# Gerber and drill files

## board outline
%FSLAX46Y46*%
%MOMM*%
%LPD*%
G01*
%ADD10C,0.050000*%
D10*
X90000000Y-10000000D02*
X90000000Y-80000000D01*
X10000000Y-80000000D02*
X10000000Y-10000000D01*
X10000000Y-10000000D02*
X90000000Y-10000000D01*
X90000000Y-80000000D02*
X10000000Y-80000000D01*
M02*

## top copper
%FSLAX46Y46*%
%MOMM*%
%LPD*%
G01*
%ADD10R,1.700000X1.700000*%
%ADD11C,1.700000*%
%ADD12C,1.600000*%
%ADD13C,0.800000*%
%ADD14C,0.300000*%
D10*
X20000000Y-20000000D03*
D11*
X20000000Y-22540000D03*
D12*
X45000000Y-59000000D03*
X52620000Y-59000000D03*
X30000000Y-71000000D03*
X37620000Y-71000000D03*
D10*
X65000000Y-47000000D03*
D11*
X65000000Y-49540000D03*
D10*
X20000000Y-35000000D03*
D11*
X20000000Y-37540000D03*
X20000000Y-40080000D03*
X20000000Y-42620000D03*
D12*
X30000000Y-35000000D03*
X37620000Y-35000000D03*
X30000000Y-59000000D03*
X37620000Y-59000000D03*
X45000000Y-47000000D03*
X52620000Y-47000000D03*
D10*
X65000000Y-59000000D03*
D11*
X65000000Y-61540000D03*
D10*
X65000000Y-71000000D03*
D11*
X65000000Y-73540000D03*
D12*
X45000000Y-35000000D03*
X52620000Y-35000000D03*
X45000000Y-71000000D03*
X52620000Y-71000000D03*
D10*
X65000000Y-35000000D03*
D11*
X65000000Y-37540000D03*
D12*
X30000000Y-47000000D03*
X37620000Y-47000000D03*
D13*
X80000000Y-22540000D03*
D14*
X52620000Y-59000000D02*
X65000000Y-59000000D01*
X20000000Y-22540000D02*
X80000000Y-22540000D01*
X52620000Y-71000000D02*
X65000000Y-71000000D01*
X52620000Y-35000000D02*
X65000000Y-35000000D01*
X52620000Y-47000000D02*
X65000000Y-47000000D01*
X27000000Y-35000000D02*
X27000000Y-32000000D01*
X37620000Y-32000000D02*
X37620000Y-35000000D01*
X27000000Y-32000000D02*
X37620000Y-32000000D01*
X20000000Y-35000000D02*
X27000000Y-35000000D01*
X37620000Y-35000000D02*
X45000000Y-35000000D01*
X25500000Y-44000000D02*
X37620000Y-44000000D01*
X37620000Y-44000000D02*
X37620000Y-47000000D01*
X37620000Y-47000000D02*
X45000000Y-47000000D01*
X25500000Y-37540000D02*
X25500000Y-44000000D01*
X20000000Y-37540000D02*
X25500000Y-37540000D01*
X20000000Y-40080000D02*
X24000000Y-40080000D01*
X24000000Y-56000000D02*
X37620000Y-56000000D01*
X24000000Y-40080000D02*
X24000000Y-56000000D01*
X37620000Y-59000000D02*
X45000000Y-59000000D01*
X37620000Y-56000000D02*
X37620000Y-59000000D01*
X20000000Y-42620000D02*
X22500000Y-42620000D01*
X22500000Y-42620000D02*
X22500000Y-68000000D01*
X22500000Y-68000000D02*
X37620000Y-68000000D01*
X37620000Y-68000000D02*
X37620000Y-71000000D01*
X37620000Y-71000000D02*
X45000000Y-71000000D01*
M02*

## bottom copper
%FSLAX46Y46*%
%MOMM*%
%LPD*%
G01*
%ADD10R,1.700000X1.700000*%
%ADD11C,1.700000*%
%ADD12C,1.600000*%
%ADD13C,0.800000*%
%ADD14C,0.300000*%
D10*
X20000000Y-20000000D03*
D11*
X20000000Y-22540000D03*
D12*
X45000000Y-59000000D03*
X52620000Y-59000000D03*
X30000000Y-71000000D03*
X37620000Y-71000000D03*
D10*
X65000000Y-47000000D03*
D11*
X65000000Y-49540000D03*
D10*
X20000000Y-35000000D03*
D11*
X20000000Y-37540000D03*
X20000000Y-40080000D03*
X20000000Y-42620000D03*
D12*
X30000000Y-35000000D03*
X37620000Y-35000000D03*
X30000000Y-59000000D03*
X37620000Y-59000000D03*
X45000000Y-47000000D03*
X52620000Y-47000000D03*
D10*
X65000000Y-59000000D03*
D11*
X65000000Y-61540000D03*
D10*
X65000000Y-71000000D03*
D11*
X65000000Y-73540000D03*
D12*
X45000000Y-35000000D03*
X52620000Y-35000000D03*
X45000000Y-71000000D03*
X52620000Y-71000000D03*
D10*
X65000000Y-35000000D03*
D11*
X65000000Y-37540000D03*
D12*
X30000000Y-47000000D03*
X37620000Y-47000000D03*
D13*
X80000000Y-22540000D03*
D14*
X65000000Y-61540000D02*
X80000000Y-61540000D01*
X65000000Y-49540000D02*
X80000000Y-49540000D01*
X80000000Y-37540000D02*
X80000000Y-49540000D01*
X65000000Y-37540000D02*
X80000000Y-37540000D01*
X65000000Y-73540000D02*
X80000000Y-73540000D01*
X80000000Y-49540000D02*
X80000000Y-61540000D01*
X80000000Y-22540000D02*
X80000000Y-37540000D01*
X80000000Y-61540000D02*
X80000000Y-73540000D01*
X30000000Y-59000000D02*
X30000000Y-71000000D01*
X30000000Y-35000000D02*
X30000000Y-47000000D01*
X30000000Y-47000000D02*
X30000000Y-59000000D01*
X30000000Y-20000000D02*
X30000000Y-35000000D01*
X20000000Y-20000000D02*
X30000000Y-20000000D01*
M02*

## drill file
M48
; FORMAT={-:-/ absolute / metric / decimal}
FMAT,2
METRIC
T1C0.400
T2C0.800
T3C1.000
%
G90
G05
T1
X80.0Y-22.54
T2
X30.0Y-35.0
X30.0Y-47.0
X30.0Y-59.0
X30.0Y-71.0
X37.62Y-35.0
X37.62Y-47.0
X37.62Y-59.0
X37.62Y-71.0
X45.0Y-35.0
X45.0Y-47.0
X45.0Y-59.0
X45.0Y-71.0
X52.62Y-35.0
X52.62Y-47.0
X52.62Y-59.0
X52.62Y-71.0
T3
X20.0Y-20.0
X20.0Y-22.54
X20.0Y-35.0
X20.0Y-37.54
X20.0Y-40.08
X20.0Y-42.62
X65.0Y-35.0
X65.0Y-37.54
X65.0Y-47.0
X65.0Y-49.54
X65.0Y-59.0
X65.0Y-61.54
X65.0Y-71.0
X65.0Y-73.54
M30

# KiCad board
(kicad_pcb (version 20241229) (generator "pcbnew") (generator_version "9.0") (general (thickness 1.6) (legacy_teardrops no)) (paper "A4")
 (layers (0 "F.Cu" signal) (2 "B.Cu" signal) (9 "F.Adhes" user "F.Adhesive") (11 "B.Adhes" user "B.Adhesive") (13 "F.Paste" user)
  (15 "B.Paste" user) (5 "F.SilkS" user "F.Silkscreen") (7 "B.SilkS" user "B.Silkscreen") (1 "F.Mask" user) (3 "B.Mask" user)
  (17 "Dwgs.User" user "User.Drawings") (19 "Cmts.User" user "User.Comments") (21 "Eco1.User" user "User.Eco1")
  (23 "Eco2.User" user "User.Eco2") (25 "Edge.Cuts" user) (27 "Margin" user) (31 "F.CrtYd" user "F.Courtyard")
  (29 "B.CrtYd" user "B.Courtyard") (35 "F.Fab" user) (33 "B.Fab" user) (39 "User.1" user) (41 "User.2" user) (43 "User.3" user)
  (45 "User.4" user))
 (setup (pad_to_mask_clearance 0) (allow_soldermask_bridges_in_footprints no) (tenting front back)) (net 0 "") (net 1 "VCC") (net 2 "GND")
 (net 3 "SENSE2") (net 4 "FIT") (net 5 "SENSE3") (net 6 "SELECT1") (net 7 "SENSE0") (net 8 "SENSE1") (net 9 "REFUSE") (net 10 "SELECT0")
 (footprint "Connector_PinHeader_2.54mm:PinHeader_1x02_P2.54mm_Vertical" (layer "F.Cu") (at 20 20)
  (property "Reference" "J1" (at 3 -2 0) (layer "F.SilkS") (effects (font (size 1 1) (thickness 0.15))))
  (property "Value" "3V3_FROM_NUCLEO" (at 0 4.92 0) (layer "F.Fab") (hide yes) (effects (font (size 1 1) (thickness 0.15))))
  (pad "1" thru_hole rect (at 0 0) (size 1.7 1.7) (drill 1) (layers "*.Cu" "*.Mask") (remove_unused_layers no) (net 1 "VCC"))
  (pad "2" thru_hole circle (at 0 2.54) (size 1.7 1.7) (drill 1) (layers "*.Cu" "*.Mask") (remove_unused_layers no) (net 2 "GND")))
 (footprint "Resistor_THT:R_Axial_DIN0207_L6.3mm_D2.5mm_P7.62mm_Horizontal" (layer "F.Cu") (at 45 59)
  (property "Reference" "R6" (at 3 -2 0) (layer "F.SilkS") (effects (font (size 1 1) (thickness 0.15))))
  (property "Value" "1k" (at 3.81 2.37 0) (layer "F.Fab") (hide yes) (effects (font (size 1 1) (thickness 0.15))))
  (pad "1" thru_hole circle (at 0 0) (size 1.6 1.6) (drill 0.8) (layers "*.Cu" "*.Mask") (remove_unused_layers no) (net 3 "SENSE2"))
  (pad "2" thru_hole circle (at 7.62 0) (size 1.6 1.6) (drill 0.8) (layers "*.Cu" "*.Mask") (remove_unused_layers no) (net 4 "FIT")))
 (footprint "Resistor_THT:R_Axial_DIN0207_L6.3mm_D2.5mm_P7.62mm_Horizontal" (layer "F.Cu") (at 30 71)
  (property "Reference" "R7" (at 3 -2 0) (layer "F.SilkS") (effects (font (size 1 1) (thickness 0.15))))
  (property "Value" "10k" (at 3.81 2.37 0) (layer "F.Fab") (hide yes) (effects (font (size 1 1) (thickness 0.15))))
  (pad "1" thru_hole circle (at 0 0) (size 1.6 1.6) (drill 0.8) (layers "*.Cu" "*.Mask") (remove_unused_layers no) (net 1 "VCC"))
  (pad "2" thru_hole circle (at 7.62 0) (size 1.6 1.6) (drill 0.8) (layers "*.Cu" "*.Mask") (remove_unused_layers no) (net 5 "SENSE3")))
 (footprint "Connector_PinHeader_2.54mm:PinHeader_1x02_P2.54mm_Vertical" (layer "F.Cu") (at 65 47)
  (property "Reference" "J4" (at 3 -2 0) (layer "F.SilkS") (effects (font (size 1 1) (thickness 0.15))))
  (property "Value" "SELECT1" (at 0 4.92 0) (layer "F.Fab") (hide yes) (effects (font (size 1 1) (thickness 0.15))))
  (pad "1" thru_hole rect (at 0 0) (size 1.7 1.7) (drill 1) (layers "*.Cu" "*.Mask") (remove_unused_layers no) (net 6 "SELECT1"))
  (pad "2" thru_hole circle (at 0 2.54) (size 1.7 1.7) (drill 1) (layers "*.Cu" "*.Mask") (remove_unused_layers no) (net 2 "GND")))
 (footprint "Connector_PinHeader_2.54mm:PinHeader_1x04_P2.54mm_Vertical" (layer "F.Cu") (at 20 35)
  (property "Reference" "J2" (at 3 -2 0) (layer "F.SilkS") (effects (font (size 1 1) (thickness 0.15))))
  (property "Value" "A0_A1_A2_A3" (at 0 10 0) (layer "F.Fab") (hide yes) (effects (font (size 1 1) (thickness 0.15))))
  (pad "1" thru_hole rect (at 0 0) (size 1.7 1.7) (drill 1) (layers "*.Cu" "*.Mask") (remove_unused_layers no) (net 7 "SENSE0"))
  (pad "2" thru_hole circle (at 0 2.54) (size 1.7 1.7) (drill 1) (layers "*.Cu" "*.Mask") (remove_unused_layers no) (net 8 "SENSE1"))
  (pad "3" thru_hole circle (at 0 5.08) (size 1.7 1.7) (drill 1) (layers "*.Cu" "*.Mask") (remove_unused_layers no) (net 3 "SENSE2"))
  (pad "4" thru_hole circle (at 0 7.62) (size 1.7 1.7) (drill 1) (layers "*.Cu" "*.Mask") (remove_unused_layers no) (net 5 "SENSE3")))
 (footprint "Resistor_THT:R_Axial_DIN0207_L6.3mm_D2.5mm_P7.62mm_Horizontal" (layer "F.Cu") (at 30 35)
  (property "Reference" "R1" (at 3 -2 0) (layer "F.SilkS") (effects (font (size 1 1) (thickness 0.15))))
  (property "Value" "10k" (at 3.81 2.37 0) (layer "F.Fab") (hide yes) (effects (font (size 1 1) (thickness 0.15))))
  (pad "1" thru_hole circle (at 0 0) (size 1.6 1.6) (drill 0.8) (layers "*.Cu" "*.Mask") (remove_unused_layers no) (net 1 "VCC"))
  (pad "2" thru_hole circle (at 7.62 0) (size 1.6 1.6) (drill 0.8) (layers "*.Cu" "*.Mask") (remove_unused_layers no) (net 7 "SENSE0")))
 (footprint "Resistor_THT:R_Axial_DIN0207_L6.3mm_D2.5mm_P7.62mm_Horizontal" (layer "F.Cu") (at 30 59)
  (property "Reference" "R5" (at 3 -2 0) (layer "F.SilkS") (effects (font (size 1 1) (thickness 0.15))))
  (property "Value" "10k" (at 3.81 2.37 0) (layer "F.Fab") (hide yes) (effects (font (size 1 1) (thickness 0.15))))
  (pad "1" thru_hole circle (at 0 0) (size 1.6 1.6) (drill 0.8) (layers "*.Cu" "*.Mask") (remove_unused_layers no) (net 1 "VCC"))
  (pad "2" thru_hole circle (at 7.62 0) (size 1.6 1.6) (drill 0.8) (layers "*.Cu" "*.Mask") (remove_unused_layers no) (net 3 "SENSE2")))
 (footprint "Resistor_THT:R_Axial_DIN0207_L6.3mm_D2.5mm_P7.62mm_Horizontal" (layer "F.Cu") (at 45 47)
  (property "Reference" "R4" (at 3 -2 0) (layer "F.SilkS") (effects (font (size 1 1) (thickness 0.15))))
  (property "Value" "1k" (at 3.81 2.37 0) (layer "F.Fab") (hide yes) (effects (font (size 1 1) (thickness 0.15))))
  (pad "1" thru_hole circle (at 0 0) (size 1.6 1.6) (drill 0.8) (layers "*.Cu" "*.Mask") (remove_unused_layers no) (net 8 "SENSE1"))
  (pad "2" thru_hole circle (at 7.62 0) (size 1.6 1.6) (drill 0.8) (layers "*.Cu" "*.Mask") (remove_unused_layers no) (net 6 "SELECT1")))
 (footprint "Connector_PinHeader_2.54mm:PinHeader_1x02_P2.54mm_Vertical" (layer "F.Cu") (at 65 59)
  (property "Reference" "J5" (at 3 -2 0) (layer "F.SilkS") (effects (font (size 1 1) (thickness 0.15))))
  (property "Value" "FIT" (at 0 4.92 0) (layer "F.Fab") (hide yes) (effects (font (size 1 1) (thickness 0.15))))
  (pad "1" thru_hole rect (at 0 0) (size 1.7 1.7) (drill 1) (layers "*.Cu" "*.Mask") (remove_unused_layers no) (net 4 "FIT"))
  (pad "2" thru_hole circle (at 0 2.54) (size 1.7 1.7) (drill 1) (layers "*.Cu" "*.Mask") (remove_unused_layers no) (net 2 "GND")))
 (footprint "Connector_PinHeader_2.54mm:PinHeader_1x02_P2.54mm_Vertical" (layer "F.Cu") (at 65 71)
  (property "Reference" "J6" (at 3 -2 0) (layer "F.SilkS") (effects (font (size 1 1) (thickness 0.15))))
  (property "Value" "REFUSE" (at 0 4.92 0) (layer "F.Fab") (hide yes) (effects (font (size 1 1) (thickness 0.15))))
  (pad "1" thru_hole rect (at 0 0) (size 1.7 1.7) (drill 1) (layers "*.Cu" "*.Mask") (remove_unused_layers no) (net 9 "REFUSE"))
  (pad "2" thru_hole circle (at 0 2.54) (size 1.7 1.7) (drill 1) (layers "*.Cu" "*.Mask") (remove_unused_layers no) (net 2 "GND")))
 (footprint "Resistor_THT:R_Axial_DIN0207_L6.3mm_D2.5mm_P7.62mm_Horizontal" (layer "F.Cu") (at 45 35)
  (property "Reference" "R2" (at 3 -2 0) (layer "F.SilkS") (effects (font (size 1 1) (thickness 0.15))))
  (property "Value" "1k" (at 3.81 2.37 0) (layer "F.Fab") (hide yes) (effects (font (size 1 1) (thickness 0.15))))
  (pad "1" thru_hole circle (at 0 0) (size 1.6 1.6) (drill 0.8) (layers "*.Cu" "*.Mask") (remove_unused_layers no) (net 7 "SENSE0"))
  (pad "2" thru_hole circle (at 7.62 0) (size 1.6 1.6) (drill 0.8) (layers "*.Cu" "*.Mask") (remove_unused_layers no) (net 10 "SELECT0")))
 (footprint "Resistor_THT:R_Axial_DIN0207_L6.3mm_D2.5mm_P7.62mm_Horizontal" (layer "F.Cu") (at 45 71)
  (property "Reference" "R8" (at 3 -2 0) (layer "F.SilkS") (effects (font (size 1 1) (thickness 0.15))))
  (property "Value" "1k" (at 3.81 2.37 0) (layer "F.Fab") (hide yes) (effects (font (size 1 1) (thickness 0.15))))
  (pad "1" thru_hole circle (at 0 0) (size 1.6 1.6) (drill 0.8) (layers "*.Cu" "*.Mask") (remove_unused_layers no) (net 5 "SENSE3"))
  (pad "2" thru_hole circle (at 7.62 0) (size 1.6 1.6) (drill 0.8) (layers "*.Cu" "*.Mask") (remove_unused_layers no) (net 9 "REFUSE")))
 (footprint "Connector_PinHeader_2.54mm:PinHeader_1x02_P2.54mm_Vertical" (layer "F.Cu") (at 65 35)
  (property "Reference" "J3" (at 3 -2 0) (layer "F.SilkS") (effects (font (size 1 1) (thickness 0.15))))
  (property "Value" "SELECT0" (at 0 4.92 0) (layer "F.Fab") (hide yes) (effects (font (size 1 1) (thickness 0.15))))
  (pad "1" thru_hole rect (at 0 0) (size 1.7 1.7) (drill 1) (layers "*.Cu" "*.Mask") (remove_unused_layers no) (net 10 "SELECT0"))
  (pad "2" thru_hole circle (at 0 2.54) (size 1.7 1.7) (drill 1) (layers "*.Cu" "*.Mask") (remove_unused_layers no) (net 2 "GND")))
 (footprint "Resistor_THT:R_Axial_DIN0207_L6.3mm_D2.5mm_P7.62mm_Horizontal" (layer "F.Cu") (at 30 47)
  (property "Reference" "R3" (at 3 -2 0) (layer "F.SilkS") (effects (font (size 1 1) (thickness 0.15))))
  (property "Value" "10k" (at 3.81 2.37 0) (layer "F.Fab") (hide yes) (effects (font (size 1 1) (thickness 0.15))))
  (pad "1" thru_hole circle (at 0 0) (size 1.6 1.6) (drill 0.8) (layers "*.Cu" "*.Mask") (remove_unused_layers no) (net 1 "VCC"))
  (pad "2" thru_hole circle (at 7.62 0) (size 1.6 1.6) (drill 0.8) (layers "*.Cu" "*.Mask") (remove_unused_layers no) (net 8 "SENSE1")))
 (gr_line (start 90 10) (end 90 80) (stroke (width 0.05) (type default)) (layer "Edge.Cuts"))
 (gr_line (start 10 80) (end 10 10) (stroke (width 0.05) (type default)) (layer "Edge.Cuts"))
 (gr_line (start 10 10) (end 90 10) (stroke (width 0.05) (type default)) (layer "Edge.Cuts"))
 (gr_line (start 90 80) (end 10 80) (stroke (width 0.05) (type default)) (layer "Edge.Cuts"))
 (segment (start 52.62 59) (end 65 59) (width 0.3) (layer "F.Cu") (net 4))
 (segment (start 20 22.54) (end 80 22.54) (width 0.3) (layer "F.Cu") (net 2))
 (via (at 80 22.54) (size 0.8) (drill 0.4) (layers "F.Cu" "B.Cu") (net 2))
 (segment (start 65 61.54) (end 80 61.54) (width 0.3) (layer "B.Cu") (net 2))
 (segment (start 65 49.54) (end 80 49.54) (width 0.3) (layer "B.Cu") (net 2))
 (segment (start 80 37.54) (end 80 49.54) (width 0.3) (layer "B.Cu") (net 2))
 (segment (start 65 37.54) (end 80 37.54) (width 0.3) (layer "B.Cu") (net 2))
 (segment (start 65 73.54) (end 80 73.54) (width 0.3) (layer "B.Cu") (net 2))
 (segment (start 80 49.54) (end 80 61.54) (width 0.3) (layer "B.Cu") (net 2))
 (segment (start 80 22.54) (end 80 37.54) (width 0.3) (layer "B.Cu") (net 2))
 (segment (start 80 61.54) (end 80 73.54) (width 0.3) (layer "B.Cu") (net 2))
 (segment (start 52.62 71) (end 65 71) (width 0.3) (layer "F.Cu") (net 9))
 (segment (start 52.62 35) (end 65 35) (width 0.3) (layer "F.Cu") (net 10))
 (segment (start 52.62 47) (end 65 47) (width 0.3) (layer "F.Cu") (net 6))
 (segment (start 27 35) (end 27 32) (width 0.3) (layer "F.Cu") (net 7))
 (segment (start 37.62 32) (end 37.62 35) (width 0.3) (layer "F.Cu") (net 7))
 (segment (start 27 32) (end 37.62 32) (width 0.3) (layer "F.Cu") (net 7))
 (segment (start 20 35) (end 27 35) (width 0.3) (layer "F.Cu") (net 7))
 (segment (start 37.62 35) (end 45 35) (width 0.3) (layer "F.Cu") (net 7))
 (segment (start 25.5 44) (end 37.62 44) (width 0.3) (layer "F.Cu") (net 8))
 (segment (start 37.62 44) (end 37.62 47) (width 0.3) (layer "F.Cu") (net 8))
 (segment (start 37.62 47) (end 45 47) (width 0.3) (layer "F.Cu") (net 8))
 (segment (start 25.5 37.54) (end 25.5 44) (width 0.3) (layer "F.Cu") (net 8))
 (segment (start 20 37.54) (end 25.5 37.54) (width 0.3) (layer "F.Cu") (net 8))
 (segment (start 20 40.08) (end 24 40.08) (width 0.3) (layer "F.Cu") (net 3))
 (segment (start 24 56) (end 37.62 56) (width 0.3) (layer "F.Cu") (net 3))
 (segment (start 24 40.08) (end 24 56) (width 0.3) (layer "F.Cu") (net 3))
 (segment (start 37.62 59) (end 45 59) (width 0.3) (layer "F.Cu") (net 3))
 (segment (start 37.62 56) (end 37.62 59) (width 0.3) (layer "F.Cu") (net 3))
 (segment (start 20 42.62) (end 22.5 42.62) (width 0.3) (layer "F.Cu") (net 5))
 (segment (start 22.5 42.62) (end 22.5 68) (width 0.3) (layer "F.Cu") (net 5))
 (segment (start 22.5 68) (end 37.62 68) (width 0.3) (layer "F.Cu") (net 5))
 (segment (start 37.62 68) (end 37.62 71) (width 0.3) (layer "F.Cu") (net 5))
 (segment (start 37.62 71) (end 45 71) (width 0.3) (layer "F.Cu") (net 5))
 (segment (start 30 59) (end 30 71) (width 0.3) (layer "B.Cu") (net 1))
 (segment (start 30 35) (end 30 47) (width 0.3) (layer "B.Cu") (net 1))
 (segment (start 30 47) (end 30 59) (width 0.3) (layer "B.Cu") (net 1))
 (segment (start 30 20) (end 30 35) (width 0.3) (layer "B.Cu") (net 1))
 (segment (start 20 20) (end 30 20) (width 0.3) (layer "B.Cu") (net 1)))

